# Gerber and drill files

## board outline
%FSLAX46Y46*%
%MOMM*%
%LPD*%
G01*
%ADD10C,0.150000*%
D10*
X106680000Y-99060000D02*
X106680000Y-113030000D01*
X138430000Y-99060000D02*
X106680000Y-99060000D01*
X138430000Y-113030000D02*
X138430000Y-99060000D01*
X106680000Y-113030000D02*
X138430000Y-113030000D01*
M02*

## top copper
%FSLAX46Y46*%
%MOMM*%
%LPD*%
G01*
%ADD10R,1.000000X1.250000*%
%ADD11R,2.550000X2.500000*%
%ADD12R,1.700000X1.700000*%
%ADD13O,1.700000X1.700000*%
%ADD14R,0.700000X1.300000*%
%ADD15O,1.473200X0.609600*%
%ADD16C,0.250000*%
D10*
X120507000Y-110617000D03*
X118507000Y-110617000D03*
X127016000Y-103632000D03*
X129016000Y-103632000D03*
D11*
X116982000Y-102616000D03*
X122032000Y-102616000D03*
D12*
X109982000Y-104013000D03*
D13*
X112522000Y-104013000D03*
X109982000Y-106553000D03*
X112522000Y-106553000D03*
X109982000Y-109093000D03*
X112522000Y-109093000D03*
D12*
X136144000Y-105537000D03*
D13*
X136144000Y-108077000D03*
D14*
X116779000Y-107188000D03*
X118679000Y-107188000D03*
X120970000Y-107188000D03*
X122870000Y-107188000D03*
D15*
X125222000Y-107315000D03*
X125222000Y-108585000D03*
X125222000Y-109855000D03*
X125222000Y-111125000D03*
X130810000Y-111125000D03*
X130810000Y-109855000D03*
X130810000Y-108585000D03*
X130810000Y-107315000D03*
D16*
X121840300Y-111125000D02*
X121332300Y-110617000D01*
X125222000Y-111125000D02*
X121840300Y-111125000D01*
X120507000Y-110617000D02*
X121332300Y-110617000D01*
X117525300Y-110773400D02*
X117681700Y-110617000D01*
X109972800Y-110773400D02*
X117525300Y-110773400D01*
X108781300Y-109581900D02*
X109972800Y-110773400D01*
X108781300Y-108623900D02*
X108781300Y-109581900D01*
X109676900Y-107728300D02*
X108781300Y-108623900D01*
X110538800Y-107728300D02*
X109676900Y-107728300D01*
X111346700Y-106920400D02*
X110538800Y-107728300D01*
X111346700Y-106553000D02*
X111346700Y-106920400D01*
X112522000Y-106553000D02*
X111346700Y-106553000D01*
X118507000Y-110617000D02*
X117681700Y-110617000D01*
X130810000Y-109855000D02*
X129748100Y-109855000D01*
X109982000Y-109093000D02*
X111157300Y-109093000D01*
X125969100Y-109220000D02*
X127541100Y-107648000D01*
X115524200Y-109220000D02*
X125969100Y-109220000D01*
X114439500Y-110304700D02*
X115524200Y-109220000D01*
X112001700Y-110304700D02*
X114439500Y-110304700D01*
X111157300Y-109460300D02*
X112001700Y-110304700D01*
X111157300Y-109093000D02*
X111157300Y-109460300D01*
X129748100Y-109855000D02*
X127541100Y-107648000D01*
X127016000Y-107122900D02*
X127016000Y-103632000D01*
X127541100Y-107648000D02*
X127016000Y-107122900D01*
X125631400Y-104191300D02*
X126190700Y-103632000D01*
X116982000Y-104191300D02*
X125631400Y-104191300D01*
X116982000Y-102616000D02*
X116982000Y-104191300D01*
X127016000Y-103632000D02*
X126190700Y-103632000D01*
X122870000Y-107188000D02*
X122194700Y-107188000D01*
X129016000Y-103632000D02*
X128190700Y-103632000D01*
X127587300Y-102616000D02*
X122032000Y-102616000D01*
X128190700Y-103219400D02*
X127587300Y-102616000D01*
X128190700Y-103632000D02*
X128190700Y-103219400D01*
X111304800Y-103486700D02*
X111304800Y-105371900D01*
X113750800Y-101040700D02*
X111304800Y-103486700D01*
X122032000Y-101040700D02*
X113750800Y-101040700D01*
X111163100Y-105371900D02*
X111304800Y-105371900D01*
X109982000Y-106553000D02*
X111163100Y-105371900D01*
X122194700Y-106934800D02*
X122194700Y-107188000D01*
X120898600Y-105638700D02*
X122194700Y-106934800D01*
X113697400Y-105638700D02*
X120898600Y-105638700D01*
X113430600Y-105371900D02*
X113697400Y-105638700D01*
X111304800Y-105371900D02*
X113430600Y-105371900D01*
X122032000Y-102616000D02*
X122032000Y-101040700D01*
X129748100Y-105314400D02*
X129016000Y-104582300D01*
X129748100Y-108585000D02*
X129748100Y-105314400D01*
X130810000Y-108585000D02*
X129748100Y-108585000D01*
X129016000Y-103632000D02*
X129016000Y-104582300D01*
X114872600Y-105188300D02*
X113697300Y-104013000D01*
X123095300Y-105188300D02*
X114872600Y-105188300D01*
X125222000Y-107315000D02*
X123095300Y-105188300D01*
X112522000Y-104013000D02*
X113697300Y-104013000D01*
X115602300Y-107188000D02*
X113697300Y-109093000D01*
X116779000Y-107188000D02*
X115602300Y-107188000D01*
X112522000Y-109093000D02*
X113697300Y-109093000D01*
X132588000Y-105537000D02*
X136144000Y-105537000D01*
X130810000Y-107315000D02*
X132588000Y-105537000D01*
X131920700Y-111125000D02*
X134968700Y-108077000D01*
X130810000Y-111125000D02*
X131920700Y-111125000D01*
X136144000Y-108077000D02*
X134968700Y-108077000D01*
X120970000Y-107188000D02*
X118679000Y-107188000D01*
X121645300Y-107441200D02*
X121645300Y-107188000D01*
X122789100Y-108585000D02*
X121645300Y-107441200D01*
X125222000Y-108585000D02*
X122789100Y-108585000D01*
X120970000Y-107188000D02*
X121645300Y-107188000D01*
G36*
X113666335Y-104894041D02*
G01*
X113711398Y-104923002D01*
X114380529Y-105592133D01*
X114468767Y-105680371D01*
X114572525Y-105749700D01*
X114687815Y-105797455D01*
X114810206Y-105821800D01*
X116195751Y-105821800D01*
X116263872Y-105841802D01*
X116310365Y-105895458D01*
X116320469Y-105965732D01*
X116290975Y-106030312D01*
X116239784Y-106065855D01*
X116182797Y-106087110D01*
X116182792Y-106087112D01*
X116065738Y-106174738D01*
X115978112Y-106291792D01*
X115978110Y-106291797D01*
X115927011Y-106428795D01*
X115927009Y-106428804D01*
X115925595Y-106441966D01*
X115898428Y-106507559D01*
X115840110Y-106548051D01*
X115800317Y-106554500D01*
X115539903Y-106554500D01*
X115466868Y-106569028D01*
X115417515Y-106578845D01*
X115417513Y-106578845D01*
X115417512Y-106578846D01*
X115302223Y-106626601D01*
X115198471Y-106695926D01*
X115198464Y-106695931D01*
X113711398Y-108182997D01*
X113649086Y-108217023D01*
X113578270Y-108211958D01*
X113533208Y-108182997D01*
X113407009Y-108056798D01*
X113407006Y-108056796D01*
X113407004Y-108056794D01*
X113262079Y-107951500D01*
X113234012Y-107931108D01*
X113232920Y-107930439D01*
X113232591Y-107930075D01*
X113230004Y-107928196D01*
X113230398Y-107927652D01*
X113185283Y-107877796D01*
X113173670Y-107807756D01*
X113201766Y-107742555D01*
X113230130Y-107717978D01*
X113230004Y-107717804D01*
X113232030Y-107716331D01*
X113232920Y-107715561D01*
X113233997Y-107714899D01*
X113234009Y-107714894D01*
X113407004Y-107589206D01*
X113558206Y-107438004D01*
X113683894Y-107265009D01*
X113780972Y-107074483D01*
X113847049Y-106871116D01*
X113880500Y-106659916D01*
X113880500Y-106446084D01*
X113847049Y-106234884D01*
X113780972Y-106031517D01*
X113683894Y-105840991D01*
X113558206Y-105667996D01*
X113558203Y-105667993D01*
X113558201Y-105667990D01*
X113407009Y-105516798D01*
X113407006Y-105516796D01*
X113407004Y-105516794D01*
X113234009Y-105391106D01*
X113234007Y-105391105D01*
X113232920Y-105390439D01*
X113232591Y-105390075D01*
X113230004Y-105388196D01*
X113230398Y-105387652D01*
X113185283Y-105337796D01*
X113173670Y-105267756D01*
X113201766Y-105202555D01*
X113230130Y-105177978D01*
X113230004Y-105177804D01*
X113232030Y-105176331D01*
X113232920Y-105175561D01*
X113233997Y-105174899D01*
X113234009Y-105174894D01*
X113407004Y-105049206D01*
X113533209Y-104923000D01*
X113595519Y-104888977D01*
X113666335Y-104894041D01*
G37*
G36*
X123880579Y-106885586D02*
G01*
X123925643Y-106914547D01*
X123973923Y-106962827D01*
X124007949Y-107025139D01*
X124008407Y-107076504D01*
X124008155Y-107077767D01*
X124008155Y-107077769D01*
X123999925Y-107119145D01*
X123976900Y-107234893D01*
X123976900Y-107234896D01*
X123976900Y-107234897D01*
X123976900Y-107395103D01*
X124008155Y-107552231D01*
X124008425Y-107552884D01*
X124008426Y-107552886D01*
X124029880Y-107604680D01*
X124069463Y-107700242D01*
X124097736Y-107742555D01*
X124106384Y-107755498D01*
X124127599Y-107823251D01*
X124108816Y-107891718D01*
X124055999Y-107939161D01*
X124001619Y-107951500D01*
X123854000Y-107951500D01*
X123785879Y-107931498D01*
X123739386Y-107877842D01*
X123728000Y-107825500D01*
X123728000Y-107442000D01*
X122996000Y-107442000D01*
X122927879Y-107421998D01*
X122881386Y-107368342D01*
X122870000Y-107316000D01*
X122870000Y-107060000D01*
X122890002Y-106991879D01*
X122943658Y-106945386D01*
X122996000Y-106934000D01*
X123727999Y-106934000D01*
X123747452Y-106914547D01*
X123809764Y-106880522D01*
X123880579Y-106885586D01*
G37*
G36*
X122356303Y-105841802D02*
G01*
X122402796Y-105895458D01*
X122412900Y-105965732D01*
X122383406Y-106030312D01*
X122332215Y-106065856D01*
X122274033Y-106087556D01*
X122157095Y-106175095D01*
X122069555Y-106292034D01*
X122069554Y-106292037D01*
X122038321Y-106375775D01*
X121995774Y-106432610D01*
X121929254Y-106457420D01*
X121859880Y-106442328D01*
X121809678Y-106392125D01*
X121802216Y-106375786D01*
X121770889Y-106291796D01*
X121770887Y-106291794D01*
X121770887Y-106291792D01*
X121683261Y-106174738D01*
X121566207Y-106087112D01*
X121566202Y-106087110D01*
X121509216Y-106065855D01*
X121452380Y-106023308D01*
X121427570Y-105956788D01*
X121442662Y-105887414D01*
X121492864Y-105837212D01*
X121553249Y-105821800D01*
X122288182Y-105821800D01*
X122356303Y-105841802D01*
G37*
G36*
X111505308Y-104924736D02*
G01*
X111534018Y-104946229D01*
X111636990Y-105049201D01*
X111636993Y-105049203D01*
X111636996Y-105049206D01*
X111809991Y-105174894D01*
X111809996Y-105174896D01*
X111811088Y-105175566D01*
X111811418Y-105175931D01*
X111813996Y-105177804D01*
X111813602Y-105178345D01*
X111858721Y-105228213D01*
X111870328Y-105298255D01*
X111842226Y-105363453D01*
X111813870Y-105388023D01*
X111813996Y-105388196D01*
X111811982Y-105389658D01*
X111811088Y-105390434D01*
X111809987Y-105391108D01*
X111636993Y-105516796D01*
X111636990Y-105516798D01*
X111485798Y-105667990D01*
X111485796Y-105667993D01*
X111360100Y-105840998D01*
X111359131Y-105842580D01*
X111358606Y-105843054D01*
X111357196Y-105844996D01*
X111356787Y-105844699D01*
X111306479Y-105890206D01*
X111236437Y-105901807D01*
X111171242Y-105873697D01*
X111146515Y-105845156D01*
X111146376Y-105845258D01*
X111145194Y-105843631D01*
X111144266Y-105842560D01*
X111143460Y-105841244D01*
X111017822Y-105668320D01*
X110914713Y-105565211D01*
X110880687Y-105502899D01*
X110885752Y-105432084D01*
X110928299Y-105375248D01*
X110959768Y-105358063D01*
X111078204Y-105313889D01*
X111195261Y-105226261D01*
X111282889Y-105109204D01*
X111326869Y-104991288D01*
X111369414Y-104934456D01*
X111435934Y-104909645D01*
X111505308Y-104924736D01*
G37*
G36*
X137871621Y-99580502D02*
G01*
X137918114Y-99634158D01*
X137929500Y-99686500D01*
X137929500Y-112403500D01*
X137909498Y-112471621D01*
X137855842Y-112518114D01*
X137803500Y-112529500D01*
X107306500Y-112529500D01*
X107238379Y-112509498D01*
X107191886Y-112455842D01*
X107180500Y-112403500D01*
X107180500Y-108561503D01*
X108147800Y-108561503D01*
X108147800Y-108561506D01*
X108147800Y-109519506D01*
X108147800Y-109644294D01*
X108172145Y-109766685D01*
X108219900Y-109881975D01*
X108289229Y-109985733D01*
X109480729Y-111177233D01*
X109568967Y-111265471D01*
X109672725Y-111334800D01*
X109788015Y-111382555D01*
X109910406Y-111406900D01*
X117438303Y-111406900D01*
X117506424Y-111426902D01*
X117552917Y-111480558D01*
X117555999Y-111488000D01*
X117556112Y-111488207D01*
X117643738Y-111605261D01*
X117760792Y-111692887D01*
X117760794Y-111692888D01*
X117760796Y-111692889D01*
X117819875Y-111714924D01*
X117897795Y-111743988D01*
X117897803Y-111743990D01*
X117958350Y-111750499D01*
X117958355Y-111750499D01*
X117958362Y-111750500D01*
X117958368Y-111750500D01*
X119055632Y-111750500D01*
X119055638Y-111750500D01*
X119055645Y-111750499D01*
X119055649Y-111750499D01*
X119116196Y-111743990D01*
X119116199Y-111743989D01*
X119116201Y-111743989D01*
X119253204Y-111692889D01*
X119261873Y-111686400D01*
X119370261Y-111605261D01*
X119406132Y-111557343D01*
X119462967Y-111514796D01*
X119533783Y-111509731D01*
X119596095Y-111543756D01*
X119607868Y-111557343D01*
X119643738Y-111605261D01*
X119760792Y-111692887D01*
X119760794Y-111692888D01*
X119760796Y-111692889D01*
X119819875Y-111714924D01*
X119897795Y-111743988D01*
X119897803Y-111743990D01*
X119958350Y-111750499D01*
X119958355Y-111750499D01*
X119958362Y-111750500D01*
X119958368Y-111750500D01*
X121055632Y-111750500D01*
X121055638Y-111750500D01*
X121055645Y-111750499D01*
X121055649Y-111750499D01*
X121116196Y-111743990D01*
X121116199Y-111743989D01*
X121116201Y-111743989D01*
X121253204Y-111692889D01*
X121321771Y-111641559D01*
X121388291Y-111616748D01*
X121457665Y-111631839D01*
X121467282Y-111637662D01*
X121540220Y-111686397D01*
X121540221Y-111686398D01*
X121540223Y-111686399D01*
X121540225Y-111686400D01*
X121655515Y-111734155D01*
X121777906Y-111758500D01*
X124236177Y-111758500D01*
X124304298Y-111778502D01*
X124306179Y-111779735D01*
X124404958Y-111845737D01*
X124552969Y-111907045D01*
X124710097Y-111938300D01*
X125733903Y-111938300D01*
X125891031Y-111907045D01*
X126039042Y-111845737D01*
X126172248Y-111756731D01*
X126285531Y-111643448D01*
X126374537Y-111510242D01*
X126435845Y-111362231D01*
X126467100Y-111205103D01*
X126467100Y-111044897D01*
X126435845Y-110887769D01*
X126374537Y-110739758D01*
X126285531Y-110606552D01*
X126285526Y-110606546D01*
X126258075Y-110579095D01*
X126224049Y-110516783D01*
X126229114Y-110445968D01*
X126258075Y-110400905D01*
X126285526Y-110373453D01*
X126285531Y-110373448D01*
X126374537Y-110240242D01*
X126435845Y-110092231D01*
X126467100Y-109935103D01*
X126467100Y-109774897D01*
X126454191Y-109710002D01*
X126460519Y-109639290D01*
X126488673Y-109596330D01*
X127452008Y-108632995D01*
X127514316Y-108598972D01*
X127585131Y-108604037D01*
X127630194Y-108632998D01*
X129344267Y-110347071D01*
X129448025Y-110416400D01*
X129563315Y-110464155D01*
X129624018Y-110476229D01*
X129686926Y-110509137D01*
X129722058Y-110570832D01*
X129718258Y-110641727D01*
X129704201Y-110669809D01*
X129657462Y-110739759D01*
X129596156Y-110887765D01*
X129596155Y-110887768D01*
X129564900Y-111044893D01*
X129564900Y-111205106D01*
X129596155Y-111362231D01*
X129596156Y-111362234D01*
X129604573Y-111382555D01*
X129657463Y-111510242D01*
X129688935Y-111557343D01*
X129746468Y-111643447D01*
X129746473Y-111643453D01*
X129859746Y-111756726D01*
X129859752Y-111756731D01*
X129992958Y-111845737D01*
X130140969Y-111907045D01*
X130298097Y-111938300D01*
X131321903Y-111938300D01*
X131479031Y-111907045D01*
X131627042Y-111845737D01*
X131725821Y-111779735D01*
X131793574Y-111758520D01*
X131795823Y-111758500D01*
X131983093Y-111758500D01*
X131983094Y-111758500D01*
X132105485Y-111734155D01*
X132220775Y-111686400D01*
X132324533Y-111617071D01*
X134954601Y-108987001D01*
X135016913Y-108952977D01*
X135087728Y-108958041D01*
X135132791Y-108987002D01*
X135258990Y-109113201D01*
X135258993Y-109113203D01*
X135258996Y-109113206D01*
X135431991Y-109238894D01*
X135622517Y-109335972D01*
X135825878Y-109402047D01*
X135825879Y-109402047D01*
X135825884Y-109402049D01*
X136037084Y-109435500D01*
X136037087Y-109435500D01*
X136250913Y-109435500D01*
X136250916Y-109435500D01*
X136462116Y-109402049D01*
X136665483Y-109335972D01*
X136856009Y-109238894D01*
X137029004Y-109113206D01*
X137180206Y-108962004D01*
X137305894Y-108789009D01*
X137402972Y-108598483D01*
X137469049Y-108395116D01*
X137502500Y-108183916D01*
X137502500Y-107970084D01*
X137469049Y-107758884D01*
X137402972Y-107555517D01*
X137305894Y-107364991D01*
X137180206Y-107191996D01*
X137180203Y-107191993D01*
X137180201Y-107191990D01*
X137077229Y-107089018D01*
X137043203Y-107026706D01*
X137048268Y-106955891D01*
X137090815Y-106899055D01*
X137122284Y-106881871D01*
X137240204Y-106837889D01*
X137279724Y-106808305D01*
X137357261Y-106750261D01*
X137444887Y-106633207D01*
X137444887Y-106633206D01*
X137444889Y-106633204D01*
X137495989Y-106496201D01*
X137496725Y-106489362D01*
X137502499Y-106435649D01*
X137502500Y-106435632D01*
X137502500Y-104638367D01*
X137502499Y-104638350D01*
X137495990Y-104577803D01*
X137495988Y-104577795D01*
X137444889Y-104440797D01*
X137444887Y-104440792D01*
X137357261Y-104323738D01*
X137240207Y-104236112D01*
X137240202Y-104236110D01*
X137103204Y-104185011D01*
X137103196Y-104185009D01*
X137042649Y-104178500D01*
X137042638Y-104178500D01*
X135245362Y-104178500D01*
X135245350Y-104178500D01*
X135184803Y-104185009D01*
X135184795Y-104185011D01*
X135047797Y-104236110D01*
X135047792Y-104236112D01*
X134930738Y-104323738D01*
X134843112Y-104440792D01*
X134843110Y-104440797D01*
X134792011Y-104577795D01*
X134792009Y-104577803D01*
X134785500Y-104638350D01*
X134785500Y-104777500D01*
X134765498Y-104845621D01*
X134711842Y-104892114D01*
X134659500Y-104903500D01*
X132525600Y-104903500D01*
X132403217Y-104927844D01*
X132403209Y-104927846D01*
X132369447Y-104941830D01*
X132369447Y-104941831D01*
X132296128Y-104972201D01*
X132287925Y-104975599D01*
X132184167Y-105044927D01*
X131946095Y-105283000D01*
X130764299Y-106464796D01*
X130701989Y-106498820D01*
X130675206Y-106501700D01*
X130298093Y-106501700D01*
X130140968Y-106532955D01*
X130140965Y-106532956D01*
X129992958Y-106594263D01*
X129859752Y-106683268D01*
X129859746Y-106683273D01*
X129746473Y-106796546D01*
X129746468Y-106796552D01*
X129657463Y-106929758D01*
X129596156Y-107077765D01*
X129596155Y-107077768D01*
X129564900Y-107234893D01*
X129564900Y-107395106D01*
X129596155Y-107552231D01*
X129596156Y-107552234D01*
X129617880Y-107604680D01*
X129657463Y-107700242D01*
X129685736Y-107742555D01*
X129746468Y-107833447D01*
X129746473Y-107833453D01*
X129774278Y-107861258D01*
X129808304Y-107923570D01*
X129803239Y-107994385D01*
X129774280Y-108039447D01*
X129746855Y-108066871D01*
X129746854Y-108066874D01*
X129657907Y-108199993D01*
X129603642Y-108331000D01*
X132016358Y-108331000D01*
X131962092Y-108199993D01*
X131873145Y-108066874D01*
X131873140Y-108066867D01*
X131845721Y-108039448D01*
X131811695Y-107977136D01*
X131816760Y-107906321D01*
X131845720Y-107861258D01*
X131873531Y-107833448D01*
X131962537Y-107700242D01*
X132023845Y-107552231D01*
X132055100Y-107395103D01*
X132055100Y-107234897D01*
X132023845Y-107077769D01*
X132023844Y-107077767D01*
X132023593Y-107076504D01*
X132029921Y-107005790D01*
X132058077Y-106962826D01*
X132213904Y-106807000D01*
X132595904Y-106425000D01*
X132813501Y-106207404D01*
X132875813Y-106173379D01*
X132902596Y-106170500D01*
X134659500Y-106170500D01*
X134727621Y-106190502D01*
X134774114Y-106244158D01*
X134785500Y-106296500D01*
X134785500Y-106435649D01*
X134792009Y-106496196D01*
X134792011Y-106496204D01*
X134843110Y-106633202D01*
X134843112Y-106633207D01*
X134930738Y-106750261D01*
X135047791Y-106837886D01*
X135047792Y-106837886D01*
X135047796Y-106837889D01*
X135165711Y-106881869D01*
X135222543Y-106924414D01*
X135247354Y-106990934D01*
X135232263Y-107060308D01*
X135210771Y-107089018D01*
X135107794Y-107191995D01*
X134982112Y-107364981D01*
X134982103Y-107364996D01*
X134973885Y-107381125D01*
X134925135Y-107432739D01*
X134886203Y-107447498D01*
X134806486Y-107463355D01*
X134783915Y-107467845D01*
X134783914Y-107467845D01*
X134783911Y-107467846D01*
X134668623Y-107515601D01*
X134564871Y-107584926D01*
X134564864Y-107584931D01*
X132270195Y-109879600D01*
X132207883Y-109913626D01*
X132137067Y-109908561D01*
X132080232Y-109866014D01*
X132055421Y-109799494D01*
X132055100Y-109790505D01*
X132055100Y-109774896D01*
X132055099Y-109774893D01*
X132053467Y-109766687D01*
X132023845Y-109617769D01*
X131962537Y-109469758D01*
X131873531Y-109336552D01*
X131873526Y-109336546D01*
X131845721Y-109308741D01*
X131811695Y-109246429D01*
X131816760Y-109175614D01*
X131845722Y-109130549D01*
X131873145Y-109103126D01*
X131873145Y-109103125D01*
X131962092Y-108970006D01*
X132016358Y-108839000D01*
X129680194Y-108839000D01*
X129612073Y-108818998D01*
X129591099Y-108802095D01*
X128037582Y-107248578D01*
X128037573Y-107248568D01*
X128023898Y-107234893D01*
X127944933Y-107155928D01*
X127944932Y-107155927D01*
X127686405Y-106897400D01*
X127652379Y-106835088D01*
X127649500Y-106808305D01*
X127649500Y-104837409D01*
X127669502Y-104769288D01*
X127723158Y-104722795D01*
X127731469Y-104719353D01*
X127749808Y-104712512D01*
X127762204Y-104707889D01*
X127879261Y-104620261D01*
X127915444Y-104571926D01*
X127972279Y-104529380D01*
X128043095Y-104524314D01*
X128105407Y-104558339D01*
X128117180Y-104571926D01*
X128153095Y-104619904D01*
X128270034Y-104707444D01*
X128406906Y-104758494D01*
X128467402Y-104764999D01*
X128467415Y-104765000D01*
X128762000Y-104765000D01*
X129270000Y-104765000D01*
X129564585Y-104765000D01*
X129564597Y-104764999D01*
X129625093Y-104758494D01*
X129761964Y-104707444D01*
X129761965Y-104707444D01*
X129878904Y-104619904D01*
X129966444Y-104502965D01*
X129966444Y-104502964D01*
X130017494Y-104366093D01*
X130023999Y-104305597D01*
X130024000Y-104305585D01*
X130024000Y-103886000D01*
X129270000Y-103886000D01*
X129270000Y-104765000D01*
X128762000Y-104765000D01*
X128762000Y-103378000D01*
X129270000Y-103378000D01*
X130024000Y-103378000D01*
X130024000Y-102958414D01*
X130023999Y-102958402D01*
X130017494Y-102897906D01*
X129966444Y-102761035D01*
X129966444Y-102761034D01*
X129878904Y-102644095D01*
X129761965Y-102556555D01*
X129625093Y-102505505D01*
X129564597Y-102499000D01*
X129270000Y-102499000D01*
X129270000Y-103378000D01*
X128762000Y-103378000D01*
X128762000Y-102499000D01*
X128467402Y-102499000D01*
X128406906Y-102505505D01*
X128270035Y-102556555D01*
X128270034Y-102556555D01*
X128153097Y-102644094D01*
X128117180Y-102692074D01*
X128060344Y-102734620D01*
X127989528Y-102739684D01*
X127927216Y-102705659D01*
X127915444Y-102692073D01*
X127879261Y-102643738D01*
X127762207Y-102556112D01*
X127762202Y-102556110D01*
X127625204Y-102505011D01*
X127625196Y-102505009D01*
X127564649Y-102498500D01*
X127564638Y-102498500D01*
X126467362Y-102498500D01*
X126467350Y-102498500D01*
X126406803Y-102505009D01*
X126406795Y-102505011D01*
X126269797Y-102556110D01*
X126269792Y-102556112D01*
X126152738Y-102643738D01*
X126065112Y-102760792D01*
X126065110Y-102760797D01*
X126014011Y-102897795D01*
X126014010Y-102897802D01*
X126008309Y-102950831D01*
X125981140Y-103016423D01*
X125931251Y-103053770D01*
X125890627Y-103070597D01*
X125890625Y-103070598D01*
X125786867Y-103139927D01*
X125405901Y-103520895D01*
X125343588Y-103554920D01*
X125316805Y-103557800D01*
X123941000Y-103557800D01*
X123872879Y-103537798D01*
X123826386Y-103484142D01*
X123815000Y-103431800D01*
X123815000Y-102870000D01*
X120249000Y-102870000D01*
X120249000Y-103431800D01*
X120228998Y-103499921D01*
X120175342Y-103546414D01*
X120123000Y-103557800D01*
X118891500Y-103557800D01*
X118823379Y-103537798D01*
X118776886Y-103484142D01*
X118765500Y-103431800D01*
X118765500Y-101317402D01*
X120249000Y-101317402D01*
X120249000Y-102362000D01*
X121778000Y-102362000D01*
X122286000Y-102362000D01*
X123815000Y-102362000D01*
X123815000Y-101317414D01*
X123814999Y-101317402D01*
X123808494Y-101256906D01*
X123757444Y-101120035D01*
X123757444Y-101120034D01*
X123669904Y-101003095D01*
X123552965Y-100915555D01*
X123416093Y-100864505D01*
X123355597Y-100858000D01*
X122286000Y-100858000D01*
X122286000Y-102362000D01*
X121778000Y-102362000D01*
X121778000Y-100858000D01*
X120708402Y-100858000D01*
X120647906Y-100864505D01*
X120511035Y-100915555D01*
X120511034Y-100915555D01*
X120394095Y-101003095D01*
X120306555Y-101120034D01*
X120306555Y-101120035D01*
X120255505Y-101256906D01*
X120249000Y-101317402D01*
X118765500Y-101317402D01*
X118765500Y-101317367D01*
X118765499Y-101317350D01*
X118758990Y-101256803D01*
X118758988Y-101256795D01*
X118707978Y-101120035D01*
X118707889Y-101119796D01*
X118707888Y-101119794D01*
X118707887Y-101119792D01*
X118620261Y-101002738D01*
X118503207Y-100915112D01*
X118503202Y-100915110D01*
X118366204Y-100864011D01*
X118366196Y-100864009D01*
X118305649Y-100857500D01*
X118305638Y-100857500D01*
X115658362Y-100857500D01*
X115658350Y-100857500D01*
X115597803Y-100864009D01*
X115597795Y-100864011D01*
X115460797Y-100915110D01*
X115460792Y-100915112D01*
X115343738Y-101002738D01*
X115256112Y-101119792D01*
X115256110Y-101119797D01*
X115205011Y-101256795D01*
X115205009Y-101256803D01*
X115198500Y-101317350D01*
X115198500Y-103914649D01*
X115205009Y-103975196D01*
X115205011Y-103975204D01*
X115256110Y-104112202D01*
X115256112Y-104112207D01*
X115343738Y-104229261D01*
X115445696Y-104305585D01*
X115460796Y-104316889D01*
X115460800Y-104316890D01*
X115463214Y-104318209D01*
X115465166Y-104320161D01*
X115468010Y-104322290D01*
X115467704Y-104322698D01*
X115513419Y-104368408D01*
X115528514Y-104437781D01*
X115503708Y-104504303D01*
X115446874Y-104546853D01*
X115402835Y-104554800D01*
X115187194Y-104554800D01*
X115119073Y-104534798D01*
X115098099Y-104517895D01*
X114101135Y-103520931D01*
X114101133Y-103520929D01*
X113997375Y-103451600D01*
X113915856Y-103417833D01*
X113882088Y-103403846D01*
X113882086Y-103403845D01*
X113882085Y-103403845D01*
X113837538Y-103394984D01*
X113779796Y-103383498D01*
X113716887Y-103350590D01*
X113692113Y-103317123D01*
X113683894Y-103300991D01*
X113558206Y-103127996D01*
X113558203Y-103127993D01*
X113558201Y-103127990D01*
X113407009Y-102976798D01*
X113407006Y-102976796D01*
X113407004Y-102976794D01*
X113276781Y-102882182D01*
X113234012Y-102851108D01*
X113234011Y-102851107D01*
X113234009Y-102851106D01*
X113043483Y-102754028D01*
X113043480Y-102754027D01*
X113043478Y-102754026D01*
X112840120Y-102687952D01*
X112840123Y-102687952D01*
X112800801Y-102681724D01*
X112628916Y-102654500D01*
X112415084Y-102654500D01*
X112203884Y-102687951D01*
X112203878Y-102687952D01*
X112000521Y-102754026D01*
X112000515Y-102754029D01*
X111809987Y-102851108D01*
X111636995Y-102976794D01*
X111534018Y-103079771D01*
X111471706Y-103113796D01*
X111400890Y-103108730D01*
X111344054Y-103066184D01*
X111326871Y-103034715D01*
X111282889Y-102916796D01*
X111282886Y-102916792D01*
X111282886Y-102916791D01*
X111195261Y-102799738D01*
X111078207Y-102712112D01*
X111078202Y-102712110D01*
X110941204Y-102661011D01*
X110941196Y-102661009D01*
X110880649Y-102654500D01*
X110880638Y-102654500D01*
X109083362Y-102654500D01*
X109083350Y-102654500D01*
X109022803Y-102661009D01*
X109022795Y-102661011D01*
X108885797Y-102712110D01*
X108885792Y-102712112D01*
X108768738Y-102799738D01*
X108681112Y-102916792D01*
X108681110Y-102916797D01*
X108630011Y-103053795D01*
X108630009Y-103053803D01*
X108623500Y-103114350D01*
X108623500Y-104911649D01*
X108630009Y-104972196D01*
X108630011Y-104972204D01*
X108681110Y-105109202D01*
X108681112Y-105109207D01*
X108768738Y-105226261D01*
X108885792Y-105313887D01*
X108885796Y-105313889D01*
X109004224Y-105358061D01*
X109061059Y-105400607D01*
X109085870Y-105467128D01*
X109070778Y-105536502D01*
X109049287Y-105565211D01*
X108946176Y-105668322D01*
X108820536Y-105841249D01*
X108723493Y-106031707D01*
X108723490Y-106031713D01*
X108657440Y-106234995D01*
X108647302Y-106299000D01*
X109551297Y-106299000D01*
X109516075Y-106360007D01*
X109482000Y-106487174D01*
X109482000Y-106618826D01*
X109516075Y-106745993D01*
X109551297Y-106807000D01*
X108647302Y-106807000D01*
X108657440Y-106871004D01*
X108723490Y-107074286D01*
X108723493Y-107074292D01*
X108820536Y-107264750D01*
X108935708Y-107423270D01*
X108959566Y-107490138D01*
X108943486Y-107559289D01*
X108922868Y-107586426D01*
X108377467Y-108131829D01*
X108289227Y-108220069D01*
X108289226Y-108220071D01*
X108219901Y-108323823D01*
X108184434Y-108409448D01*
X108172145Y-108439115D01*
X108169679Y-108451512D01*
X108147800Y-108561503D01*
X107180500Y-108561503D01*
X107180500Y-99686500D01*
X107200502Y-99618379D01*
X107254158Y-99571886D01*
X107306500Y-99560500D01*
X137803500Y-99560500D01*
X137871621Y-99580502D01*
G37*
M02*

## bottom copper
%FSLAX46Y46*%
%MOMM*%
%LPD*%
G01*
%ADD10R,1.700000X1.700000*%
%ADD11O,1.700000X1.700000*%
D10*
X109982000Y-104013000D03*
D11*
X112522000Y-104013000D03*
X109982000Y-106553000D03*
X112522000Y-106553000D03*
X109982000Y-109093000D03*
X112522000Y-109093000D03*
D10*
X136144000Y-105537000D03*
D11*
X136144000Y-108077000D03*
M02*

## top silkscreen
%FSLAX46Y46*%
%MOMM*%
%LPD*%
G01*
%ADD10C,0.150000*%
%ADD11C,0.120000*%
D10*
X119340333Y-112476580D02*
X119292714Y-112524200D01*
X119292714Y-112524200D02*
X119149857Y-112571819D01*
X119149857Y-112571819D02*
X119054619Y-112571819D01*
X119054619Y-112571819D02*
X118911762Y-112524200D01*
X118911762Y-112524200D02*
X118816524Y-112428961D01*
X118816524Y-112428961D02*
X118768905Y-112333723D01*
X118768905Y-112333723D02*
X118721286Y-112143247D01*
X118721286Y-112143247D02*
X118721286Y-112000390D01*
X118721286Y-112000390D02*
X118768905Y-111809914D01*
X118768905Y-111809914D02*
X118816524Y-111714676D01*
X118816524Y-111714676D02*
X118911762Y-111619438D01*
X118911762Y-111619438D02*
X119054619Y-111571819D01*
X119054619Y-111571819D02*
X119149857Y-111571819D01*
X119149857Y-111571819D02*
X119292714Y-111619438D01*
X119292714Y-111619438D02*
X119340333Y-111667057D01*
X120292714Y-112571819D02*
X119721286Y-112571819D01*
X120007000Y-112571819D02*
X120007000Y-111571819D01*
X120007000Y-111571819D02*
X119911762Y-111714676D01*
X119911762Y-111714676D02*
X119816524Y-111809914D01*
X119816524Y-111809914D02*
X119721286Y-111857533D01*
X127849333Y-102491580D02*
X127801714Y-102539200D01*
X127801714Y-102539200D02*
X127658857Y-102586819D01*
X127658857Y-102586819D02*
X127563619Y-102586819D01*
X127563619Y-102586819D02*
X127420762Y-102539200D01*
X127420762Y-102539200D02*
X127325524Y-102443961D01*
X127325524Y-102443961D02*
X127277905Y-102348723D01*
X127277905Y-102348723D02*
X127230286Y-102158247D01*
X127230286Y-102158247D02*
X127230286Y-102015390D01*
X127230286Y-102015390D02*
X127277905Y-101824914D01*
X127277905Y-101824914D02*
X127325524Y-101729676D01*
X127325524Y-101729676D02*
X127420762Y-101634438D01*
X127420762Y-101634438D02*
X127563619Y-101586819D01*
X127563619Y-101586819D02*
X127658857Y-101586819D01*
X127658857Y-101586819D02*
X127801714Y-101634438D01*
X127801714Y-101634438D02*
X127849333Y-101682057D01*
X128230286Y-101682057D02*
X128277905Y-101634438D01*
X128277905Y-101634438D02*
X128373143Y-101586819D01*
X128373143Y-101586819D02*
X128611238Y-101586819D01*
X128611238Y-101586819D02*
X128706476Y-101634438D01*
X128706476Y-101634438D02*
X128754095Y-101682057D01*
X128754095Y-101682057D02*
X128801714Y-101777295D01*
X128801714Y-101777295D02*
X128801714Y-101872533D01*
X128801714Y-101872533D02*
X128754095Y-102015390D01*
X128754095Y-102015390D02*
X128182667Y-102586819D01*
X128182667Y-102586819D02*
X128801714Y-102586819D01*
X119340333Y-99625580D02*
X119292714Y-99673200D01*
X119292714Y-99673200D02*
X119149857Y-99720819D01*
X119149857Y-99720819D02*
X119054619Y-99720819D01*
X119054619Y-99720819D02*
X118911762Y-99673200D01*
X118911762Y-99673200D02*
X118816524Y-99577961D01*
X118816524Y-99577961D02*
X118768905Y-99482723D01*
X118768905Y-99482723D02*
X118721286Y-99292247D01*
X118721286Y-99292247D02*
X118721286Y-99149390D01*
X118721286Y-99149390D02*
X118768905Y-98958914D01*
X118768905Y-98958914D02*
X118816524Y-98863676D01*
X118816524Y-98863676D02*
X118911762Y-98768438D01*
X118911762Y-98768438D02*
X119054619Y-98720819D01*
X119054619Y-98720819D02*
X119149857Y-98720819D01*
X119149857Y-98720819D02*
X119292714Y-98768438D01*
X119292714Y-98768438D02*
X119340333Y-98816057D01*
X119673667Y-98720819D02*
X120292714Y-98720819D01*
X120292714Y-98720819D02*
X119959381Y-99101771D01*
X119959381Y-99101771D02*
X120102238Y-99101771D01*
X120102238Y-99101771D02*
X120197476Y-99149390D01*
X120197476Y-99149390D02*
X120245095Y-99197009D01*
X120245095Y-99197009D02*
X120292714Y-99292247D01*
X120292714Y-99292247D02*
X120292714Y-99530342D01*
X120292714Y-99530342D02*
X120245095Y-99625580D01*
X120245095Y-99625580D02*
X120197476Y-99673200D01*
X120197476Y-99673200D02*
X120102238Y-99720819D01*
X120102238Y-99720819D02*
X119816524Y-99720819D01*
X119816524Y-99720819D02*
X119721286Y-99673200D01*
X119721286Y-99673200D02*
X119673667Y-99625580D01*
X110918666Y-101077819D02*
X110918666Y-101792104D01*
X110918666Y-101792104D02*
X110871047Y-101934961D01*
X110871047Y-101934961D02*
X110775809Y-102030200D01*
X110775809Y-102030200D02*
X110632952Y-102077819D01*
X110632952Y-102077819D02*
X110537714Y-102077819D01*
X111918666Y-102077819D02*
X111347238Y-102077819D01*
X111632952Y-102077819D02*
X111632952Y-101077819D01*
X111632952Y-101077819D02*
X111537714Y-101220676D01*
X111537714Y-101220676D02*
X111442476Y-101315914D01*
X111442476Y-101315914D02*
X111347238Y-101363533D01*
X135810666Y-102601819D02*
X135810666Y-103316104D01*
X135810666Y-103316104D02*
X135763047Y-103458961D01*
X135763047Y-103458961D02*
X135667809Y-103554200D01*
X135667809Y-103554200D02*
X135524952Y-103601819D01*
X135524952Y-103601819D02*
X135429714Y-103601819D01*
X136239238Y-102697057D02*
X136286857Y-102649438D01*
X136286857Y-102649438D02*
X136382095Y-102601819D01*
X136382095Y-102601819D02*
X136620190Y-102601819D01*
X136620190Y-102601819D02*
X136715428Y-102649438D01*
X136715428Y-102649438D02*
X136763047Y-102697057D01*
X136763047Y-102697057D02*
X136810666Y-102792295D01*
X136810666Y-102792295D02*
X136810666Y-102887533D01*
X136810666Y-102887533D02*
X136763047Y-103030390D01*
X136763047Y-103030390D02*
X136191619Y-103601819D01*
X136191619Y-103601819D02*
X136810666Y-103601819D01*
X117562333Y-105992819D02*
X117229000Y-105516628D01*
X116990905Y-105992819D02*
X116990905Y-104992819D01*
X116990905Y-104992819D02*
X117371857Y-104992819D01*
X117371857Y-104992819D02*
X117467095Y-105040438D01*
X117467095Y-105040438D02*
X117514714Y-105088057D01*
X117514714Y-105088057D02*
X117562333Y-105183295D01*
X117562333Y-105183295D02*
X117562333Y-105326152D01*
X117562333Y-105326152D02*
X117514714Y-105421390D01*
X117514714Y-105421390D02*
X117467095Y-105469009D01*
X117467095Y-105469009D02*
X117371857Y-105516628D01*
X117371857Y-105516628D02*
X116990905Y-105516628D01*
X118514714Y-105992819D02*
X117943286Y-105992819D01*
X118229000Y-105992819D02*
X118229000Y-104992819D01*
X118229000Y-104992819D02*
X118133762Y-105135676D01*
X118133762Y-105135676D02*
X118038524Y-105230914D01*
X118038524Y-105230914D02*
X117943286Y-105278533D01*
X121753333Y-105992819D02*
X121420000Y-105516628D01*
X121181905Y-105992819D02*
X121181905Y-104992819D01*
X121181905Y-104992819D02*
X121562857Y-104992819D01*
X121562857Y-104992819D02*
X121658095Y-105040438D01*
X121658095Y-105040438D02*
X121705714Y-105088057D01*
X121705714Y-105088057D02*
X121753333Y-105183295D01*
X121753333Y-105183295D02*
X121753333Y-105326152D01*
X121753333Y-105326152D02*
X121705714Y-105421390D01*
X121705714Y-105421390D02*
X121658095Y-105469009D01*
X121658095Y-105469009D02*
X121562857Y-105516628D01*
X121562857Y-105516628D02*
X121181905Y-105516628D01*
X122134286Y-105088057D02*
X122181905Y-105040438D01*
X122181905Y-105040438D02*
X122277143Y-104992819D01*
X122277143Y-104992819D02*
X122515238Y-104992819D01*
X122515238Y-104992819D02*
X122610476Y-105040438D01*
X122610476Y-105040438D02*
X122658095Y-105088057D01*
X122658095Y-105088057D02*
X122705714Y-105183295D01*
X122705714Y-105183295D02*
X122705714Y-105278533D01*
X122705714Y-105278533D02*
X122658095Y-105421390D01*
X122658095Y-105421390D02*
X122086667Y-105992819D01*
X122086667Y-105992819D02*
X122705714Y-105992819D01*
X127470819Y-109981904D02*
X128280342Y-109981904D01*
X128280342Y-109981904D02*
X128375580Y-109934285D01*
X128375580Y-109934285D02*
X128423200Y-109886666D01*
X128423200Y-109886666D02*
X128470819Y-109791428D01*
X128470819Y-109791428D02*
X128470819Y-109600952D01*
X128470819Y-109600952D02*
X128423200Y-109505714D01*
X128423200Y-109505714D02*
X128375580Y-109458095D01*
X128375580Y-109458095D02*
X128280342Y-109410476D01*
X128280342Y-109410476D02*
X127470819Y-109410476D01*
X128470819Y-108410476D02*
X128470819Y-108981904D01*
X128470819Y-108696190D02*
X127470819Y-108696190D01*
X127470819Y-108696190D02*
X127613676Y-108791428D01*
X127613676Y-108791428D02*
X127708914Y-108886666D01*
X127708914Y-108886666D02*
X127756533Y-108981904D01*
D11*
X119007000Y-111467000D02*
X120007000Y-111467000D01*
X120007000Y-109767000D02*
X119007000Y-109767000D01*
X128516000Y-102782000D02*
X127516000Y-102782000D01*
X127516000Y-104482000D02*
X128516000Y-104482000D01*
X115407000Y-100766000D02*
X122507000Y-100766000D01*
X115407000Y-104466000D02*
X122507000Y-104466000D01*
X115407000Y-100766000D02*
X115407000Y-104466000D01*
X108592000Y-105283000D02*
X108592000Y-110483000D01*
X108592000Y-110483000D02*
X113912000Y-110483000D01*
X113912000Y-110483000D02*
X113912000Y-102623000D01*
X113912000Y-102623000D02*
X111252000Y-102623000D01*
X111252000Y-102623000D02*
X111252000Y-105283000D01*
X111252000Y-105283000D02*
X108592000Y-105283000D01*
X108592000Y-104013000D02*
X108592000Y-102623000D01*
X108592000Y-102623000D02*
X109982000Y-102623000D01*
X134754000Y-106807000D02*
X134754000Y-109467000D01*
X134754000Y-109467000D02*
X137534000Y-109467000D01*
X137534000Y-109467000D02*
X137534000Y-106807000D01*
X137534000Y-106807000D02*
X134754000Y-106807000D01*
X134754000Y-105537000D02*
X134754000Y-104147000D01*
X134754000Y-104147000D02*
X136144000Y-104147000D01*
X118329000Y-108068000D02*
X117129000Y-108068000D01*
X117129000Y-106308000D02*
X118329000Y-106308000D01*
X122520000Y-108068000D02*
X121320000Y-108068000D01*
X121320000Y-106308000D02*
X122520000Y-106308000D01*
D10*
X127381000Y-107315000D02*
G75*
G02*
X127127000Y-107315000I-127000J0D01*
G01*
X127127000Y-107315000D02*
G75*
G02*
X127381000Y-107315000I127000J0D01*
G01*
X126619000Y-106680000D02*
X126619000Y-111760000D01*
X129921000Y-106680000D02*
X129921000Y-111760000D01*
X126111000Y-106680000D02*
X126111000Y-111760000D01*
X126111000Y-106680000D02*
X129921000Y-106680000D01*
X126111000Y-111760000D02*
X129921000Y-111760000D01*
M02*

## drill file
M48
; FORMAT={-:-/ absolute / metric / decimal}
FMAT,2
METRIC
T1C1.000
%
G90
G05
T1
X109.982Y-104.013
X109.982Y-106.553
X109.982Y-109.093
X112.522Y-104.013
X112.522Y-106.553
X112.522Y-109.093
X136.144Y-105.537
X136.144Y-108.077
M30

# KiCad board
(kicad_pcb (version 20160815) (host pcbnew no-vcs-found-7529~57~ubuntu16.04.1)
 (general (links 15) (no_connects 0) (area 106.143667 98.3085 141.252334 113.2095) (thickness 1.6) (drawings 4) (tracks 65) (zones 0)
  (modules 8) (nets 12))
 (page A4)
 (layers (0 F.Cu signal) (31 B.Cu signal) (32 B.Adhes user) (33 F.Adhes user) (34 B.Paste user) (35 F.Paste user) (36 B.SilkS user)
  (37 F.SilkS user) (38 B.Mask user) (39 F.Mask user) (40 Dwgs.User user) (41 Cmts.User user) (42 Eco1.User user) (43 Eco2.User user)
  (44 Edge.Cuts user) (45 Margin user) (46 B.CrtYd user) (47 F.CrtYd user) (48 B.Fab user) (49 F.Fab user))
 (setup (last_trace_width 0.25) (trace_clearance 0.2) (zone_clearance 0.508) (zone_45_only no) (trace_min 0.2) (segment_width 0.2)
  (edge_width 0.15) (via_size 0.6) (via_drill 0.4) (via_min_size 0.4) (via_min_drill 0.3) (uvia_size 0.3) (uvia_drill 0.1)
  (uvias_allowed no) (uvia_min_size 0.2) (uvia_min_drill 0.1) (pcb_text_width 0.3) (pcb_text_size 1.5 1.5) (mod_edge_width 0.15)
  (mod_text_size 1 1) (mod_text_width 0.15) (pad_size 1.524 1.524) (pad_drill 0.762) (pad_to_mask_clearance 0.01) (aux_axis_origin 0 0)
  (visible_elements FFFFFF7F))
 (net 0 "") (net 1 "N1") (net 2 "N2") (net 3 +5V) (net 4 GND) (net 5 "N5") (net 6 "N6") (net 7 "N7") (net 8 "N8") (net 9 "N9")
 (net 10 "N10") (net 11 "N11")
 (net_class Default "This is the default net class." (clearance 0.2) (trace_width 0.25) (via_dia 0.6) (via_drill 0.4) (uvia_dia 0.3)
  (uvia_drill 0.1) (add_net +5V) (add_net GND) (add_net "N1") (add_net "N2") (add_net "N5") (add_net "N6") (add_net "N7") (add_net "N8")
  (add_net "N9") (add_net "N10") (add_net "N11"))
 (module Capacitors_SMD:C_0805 (layer F.Cu) (at 119.507 110.617 180)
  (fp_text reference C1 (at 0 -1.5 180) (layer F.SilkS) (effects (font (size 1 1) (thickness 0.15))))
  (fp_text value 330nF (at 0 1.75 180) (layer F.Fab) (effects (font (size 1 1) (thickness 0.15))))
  (fp_line (start 0.5 -0.85) (end -0.5 -0.85) (layer F.SilkS) (width 0.12))
  (fp_line (start -0.5 0.85) (end 0.5 0.85) (layer F.SilkS) (width 0.12))
  (pad 1 smd rect (at -1 0 180) (size 1 1.25) (layers F.Cu F.Paste F.Mask) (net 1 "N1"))
  (pad 2 smd rect (at 1 0 180) (size 1 1.25) (layers F.Cu F.Paste F.Mask) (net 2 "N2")))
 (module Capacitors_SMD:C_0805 (layer F.Cu) (at 128.016 103.632)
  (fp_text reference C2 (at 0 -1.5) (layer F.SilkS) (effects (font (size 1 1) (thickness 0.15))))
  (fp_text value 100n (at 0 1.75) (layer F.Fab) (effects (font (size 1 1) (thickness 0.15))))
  (fp_line (start 0.5 -0.85) (end -0.5 -0.85) (layer F.SilkS) (width 0.12))
  (fp_line (start -0.5 0.85) (end 0.5 0.85) (layer F.SilkS) (width 0.12))
  (pad 1 smd rect (at -1 0) (size 1 1.25) (layers F.Cu F.Paste F.Mask) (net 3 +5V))
  (pad 2 smd rect (at 1 0) (size 1 1.25) (layers F.Cu F.Paste F.Mask) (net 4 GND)))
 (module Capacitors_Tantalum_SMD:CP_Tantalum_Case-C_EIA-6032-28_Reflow (layer F.Cu) (at 119.507 102.616)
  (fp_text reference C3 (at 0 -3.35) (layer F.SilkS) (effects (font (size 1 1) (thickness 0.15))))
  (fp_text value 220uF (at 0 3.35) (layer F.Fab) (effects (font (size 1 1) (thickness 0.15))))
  (fp_line (start -4.1 -1.85) (end 3 -1.85) (layer F.SilkS) (width 0.12))
  (fp_line (start -4.1 1.85) (end 3 1.85) (layer F.SilkS) (width 0.12))
  (fp_line (start -4.1 -1.85) (end -4.1 1.85) (layer F.SilkS) (width 0.12))
  (pad 1 smd rect (at -2.525 0) (size 2.55 2.5) (layers F.Cu F.Paste F.Mask) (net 3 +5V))
  (pad 2 smd rect (at 2.525 0) (size 2.55 2.5) (layers F.Cu F.Paste F.Mask) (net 4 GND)))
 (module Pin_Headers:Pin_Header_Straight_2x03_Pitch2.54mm (layer F.Cu) (at 109.982 104.013)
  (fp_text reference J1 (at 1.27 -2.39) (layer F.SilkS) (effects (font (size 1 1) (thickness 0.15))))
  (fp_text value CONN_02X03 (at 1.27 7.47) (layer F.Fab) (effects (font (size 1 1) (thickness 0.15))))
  (fp_line (start -1.39 1.27) (end -1.39 6.47) (layer F.SilkS) (width 0.12))
  (fp_line (start -1.39 6.47) (end 3.93 6.47) (layer F.SilkS) (width 0.12))
  (fp_line (start 3.93 6.47) (end 3.93 -1.39) (layer F.SilkS) (width 0.12))
  (fp_line (start 3.93 -1.39) (end 1.27 -1.39) (layer F.SilkS) (width 0.12))
  (fp_line (start 1.27 -1.39) (end 1.27 1.27) (layer F.SilkS) (width 0.12))
  (fp_line (start 1.27 1.27) (end -1.39 1.27) (layer F.SilkS) (width 0.12))
  (fp_line (start -1.39 0) (end -1.39 -1.39) (layer F.SilkS) (width 0.12))
  (fp_line (start -1.39 -1.39) (end 0 -1.39) (layer F.SilkS) (width 0.12))
  (pad 1 thru_hole rect (at 0 0) (size 1.7 1.7) (drill 1) (layers *.Cu *.Mask) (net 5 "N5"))
  (pad 2 thru_hole oval (at 2.54 0) (size 1.7 1.7) (drill 1) (layers *.Cu *.Mask) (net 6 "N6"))
  (pad 3 thru_hole oval (at 0 2.54) (size 1.7 1.7) (drill 1) (layers *.Cu *.Mask) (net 4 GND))
  (pad 4 thru_hole oval (at 2.54 2.54) (size 1.7 1.7) (drill 1) (layers *.Cu *.Mask) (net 2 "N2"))
  (pad 5 thru_hole oval (at 0 5.08) (size 1.7 1.7) (drill 1) (layers *.Cu *.Mask) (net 3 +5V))
  (pad 6 thru_hole oval (at 2.54 5.08) (size 1.7 1.7) (drill 1) (layers *.Cu *.Mask) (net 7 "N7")))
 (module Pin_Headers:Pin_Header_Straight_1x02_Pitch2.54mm (layer F.Cu) (at 136.144 105.537)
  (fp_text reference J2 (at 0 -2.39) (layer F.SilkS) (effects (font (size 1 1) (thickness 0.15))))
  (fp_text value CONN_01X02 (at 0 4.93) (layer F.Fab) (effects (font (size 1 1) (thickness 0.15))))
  (fp_line (start -1.39 1.27) (end -1.39 3.93) (layer F.SilkS) (width 0.12))
  (fp_line (start -1.39 3.93) (end 1.39 3.93) (layer F.SilkS) (width 0.12))
  (fp_line (start 1.39 3.93) (end 1.39 1.27) (layer F.SilkS) (width 0.12))
  (fp_line (start 1.39 1.27) (end -1.39 1.27) (layer F.SilkS) (width 0.12))
  (fp_line (start -1.39 0) (end -1.39 -1.39) (layer F.SilkS) (width 0.12))
  (fp_line (start -1.39 -1.39) (end 0 -1.39) (layer F.SilkS) (width 0.12))
  (pad 1 thru_hole rect (at 0 0) (size 1.7 1.7) (drill 1) (layers *.Cu *.Mask) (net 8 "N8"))
  (pad 2 thru_hole oval (at 0 2.54) (size 1.7 1.7) (drill 1) (layers *.Cu *.Mask) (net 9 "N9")))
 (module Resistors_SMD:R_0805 (layer F.Cu) (at 117.729 107.188)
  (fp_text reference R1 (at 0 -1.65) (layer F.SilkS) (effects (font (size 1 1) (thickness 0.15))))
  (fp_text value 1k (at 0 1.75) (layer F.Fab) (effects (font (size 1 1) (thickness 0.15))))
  (fp_line (start 0.6 0.88) (end -0.6 0.88) (layer F.SilkS) (width 0.12))
  (fp_line (start -0.6 -0.88) (end 0.6 -0.88) (layer F.SilkS) (width 0.12))
  (pad 1 smd rect (at -0.95 0) (size 0.7 1.3) (layers F.Cu F.Paste F.Mask) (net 7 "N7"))
  (pad 2 smd rect (at 0.95 0) (size 0.7 1.3) (layers F.Cu F.Paste F.Mask) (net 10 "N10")))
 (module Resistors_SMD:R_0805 (layer F.Cu) (at 121.92 107.188)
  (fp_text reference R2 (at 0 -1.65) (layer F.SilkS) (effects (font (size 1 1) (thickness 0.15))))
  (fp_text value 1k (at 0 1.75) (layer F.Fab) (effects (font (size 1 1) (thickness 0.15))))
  (fp_line (start 0.6 0.88) (end -0.6 0.88) (layer F.SilkS) (width 0.12))
  (fp_line (start -0.6 -0.88) (end 0.6 -0.88) (layer F.SilkS) (width 0.12))
  (pad 1 smd rect (at -0.95 0) (size 0.7 1.3) (layers F.Cu F.Paste F.Mask) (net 10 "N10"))
  (pad 2 smd rect (at 0.95 0) (size 0.7 1.3) (layers F.Cu F.Paste F.Mask) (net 4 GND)))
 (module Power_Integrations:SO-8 (layer F.Cu) (at 128.016 109.22 270)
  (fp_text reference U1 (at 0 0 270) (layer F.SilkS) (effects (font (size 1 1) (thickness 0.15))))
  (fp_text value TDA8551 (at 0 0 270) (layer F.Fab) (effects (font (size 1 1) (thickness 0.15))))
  (fp_circle (center -1.905 0.762) (end -1.778 0.762) (layer F.SilkS) (width 0.15))
  (fp_line (start -2.54 1.397) (end 2.54 1.397) (layer F.SilkS) (width 0.15))
  (fp_line (start -2.54 -1.905) (end 2.54 -1.905) (layer F.SilkS) (width 0.15))
  (fp_line (start -2.54 1.905) (end 2.54 1.905) (layer F.SilkS) (width 0.15))
  (fp_line (start -2.54 1.905) (end -2.54 -1.905) (layer F.SilkS) (width 0.15))
  (fp_line (start 2.54 1.905) (end 2.54 -1.905) (layer F.SilkS) (width 0.15))
  (pad 1 smd oval (at -1.905 2.794 270) (size 0.6096 1.4732) (layers F.Cu F.Paste F.Mask) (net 6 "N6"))
  (pad 2 smd oval (at -0.635 2.794 270) (size 0.6096 1.4732) (layers F.Cu F.Paste F.Mask) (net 10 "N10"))
  (pad 3 smd oval (at 0.635 2.794 270) (size 0.6096 1.4732) (layers F.Cu F.Paste F.Mask) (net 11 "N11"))
  (pad 4 smd oval (at 1.905 2.794 270) (size 0.6096 1.4732) (layers F.Cu F.Paste F.Mask) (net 1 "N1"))
  (pad 5 smd oval (at 1.905 -2.794 270) (size 0.6096 1.4732) (layers F.Cu F.Paste F.Mask) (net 9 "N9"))
  (pad 6 smd oval (at 0.635 -2.794 270) (size 0.6096 1.4732) (layers F.Cu F.Paste F.Mask) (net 3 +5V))
  (pad 7 smd oval (at -0.635 -2.794 270) (size 0.6096 1.4732) (layers F.Cu F.Paste F.Mask) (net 4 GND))
  (pad 8 smd oval (at -1.905 -2.794 270) (size 0.6096 1.4732) (layers F.Cu F.Paste F.Mask) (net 8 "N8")))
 (gr_line (start 106.68 99.06) (end 106.68 113.03) (angle 90) (layer Edge.Cuts) (width 0.15))
 (gr_line (start 138.43 99.06) (end 106.68 99.06) (angle 90) (layer Edge.Cuts) (width 0.15))
 (gr_line (start 138.43 113.03) (end 138.43 99.06) (angle 90) (layer Edge.Cuts) (width 0.15))
 (gr_line (start 106.68 113.03) (end 138.43 113.03) (angle 90) (layer Edge.Cuts) (width 0.15))
 (segment (start 121.8403 111.125) (end 121.3323 110.617) (width 0.25) (layer F.Cu) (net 1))
 (segment (start 125.222 111.125) (end 121.8403 111.125) (width 0.25) (layer F.Cu) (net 1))
 (segment (start 120.507 110.617) (end 121.3323 110.617) (width 0.25) (layer F.Cu) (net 1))
 (segment (start 117.5253 110.7734) (end 117.6817 110.617) (width 0.25) (layer F.Cu) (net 2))
 (segment (start 109.9728 110.7734) (end 117.5253 110.7734) (width 0.25) (layer F.Cu) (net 2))
 (segment (start 108.7813 109.5819) (end 109.9728 110.7734) (width 0.25) (layer F.Cu) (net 2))
 (segment (start 108.7813 108.6239) (end 108.7813 109.5819) (width 0.25) (layer F.Cu) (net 2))
 (segment (start 109.6769 107.7283) (end 108.7813 108.6239) (width 0.25) (layer F.Cu) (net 2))
 (segment (start 110.5388 107.7283) (end 109.6769 107.7283) (width 0.25) (layer F.Cu) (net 2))
 (segment (start 111.3467 106.9204) (end 110.5388 107.7283) (width 0.25) (layer F.Cu) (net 2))
 (segment (start 111.3467 106.553) (end 111.3467 106.9204) (width 0.25) (layer F.Cu) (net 2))
 (segment (start 112.522 106.553) (end 111.3467 106.553) (width 0.25) (layer F.Cu) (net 2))
 (segment (start 118.507 110.617) (end 117.6817 110.617) (width 0.25) (layer F.Cu) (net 2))
 (segment (start 130.81 109.855) (end 129.7481 109.855) (width 0.25) (layer F.Cu) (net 3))
 (segment (start 109.982 109.093) (end 111.1573 109.093) (width 0.25) (layer F.Cu) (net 3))
 (segment (start 125.9691 109.22) (end 127.5411 107.648) (width 0.25) (layer F.Cu) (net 3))
 (segment (start 115.5242 109.22) (end 125.9691 109.22) (width 0.25) (layer F.Cu) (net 3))
 (segment (start 114.4395 110.3047) (end 115.5242 109.22) (width 0.25) (layer F.Cu) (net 3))
 (segment (start 112.0017 110.3047) (end 114.4395 110.3047) (width 0.25) (layer F.Cu) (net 3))
 (segment (start 111.1573 109.4603) (end 112.0017 110.3047) (width 0.25) (layer F.Cu) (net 3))
 (segment (start 111.1573 109.093) (end 111.1573 109.4603) (width 0.25) (layer F.Cu) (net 3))
 (segment (start 129.7481 109.855) (end 127.5411 107.648) (width 0.25) (layer F.Cu) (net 3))
 (segment (start 127.016 107.1229) (end 127.016 103.632) (width 0.25) (layer F.Cu) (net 3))
 (segment (start 127.5411 107.648) (end 127.016 107.1229) (width 0.25) (layer F.Cu) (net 3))
 (segment (start 125.6314 104.1913) (end 126.1907 103.632) (width 0.25) (layer F.Cu) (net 3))
 (segment (start 116.982 104.1913) (end 125.6314 104.1913) (width 0.25) (layer F.Cu) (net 3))
 (segment (start 116.982 102.616) (end 116.982 104.1913) (width 0.25) (layer F.Cu) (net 3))
 (segment (start 127.016 103.632) (end 126.1907 103.632) (width 0.25) (layer F.Cu) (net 3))
 (segment (start 122.87 107.188) (end 122.1947 107.188) (width 0.25) (layer F.Cu) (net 4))
 (segment (start 129.016 103.632) (end 128.1907 103.632) (width 0.25) (layer F.Cu) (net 4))
 (segment (start 127.5873 102.616) (end 122.032 102.616) (width 0.25) (layer F.Cu) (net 4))
 (segment (start 128.1907 103.2194) (end 127.5873 102.616) (width 0.25) (layer F.Cu) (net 4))
 (segment (start 128.1907 103.632) (end 128.1907 103.2194) (width 0.25) (layer F.Cu) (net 4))
 (segment (start 111.3048 103.4867) (end 111.3048 105.3719) (width 0.25) (layer F.Cu) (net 4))
 (segment (start 113.7508 101.0407) (end 111.3048 103.4867) (width 0.25) (layer F.Cu) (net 4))
 (segment (start 122.032 101.0407) (end 113.7508 101.0407) (width 0.25) (layer F.Cu) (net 4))
 (segment (start 111.1631 105.3719) (end 111.3048 105.3719) (width 0.25) (layer F.Cu) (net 4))
 (segment (start 109.982 106.553) (end 111.1631 105.3719) (width 0.25) (layer F.Cu) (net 4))
 (segment (start 122.1947 106.9348) (end 122.1947 107.188) (width 0.25) (layer F.Cu) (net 4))
 (segment (start 120.8986 105.6387) (end 122.1947 106.9348) (width 0.25) (layer F.Cu) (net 4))
 (segment (start 113.6974 105.6387) (end 120.8986 105.6387) (width 0.25) (layer F.Cu) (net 4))
 (segment (start 113.4306 105.3719) (end 113.6974 105.6387) (width 0.25) (layer F.Cu) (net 4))
 (segment (start 111.3048 105.3719) (end 113.4306 105.3719) (width 0.25) (layer F.Cu) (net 4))
 (segment (start 122.032 102.616) (end 122.032 101.0407) (width 0.25) (layer F.Cu) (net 4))
 (segment (start 129.7481 105.3144) (end 129.016 104.5823) (width 0.25) (layer F.Cu) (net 4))
 (segment (start 129.7481 108.585) (end 129.7481 105.3144) (width 0.25) (layer F.Cu) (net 4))
 (segment (start 130.81 108.585) (end 129.7481 108.585) (width 0.25) (layer F.Cu) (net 4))
 (segment (start 129.016 103.632) (end 129.016 104.5823) (width 0.25) (layer F.Cu) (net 4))
 (segment (start 114.8726 105.1883) (end 113.6973 104.013) (width 0.25) (layer F.Cu) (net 6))
 (segment (start 123.0953 105.1883) (end 114.8726 105.1883) (width 0.25) (layer F.Cu) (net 6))
 (segment (start 125.222 107.315) (end 123.0953 105.1883) (width 0.25) (layer F.Cu) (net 6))
 (segment (start 112.522 104.013) (end 113.6973 104.013) (width 0.25) (layer F.Cu) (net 6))
 (segment (start 115.6023 107.188) (end 113.6973 109.093) (width 0.25) (layer F.Cu) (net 7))
 (segment (start 116.779 107.188) (end 115.6023 107.188) (width 0.25) (layer F.Cu) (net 7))
 (segment (start 112.522 109.093) (end 113.6973 109.093) (width 0.25) (layer F.Cu) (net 7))
 (segment (start 132.588 105.537) (end 136.144 105.537) (width 0.25) (layer F.Cu) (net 8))
 (segment (start 130.81 107.315) (end 132.588 105.537) (width 0.25) (layer F.Cu) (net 8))
 (segment (start 131.9207 111.125) (end 134.9687 108.077) (width 0.25) (layer F.Cu) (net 9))
 (segment (start 130.81 111.125) (end 131.9207 111.125) (width 0.25) (layer F.Cu) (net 9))
 (segment (start 136.144 108.077) (end 134.9687 108.077) (width 0.25) (layer F.Cu) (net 9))
 (segment (start 120.97 107.188) (end 118.679 107.188) (width 0.25) (layer F.Cu) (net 10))
 (segment (start 121.6453 107.4412) (end 121.6453 107.188) (width 0.25) (layer F.Cu) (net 10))
 (segment (start 122.7891 108.585) (end 121.6453 107.4412) (width 0.25) (layer F.Cu) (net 10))
 (segment (start 125.222 108.585) (end 122.7891 108.585) (width 0.25) (layer F.Cu) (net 10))
 (segment (start 120.97 107.188) (end 121.6453 107.188) (width 0.25) (layer F.Cu) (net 10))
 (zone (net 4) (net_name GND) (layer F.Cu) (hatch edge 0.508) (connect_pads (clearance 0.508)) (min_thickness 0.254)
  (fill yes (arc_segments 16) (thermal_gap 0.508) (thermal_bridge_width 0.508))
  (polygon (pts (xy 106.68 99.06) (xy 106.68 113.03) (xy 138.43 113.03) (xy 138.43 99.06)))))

